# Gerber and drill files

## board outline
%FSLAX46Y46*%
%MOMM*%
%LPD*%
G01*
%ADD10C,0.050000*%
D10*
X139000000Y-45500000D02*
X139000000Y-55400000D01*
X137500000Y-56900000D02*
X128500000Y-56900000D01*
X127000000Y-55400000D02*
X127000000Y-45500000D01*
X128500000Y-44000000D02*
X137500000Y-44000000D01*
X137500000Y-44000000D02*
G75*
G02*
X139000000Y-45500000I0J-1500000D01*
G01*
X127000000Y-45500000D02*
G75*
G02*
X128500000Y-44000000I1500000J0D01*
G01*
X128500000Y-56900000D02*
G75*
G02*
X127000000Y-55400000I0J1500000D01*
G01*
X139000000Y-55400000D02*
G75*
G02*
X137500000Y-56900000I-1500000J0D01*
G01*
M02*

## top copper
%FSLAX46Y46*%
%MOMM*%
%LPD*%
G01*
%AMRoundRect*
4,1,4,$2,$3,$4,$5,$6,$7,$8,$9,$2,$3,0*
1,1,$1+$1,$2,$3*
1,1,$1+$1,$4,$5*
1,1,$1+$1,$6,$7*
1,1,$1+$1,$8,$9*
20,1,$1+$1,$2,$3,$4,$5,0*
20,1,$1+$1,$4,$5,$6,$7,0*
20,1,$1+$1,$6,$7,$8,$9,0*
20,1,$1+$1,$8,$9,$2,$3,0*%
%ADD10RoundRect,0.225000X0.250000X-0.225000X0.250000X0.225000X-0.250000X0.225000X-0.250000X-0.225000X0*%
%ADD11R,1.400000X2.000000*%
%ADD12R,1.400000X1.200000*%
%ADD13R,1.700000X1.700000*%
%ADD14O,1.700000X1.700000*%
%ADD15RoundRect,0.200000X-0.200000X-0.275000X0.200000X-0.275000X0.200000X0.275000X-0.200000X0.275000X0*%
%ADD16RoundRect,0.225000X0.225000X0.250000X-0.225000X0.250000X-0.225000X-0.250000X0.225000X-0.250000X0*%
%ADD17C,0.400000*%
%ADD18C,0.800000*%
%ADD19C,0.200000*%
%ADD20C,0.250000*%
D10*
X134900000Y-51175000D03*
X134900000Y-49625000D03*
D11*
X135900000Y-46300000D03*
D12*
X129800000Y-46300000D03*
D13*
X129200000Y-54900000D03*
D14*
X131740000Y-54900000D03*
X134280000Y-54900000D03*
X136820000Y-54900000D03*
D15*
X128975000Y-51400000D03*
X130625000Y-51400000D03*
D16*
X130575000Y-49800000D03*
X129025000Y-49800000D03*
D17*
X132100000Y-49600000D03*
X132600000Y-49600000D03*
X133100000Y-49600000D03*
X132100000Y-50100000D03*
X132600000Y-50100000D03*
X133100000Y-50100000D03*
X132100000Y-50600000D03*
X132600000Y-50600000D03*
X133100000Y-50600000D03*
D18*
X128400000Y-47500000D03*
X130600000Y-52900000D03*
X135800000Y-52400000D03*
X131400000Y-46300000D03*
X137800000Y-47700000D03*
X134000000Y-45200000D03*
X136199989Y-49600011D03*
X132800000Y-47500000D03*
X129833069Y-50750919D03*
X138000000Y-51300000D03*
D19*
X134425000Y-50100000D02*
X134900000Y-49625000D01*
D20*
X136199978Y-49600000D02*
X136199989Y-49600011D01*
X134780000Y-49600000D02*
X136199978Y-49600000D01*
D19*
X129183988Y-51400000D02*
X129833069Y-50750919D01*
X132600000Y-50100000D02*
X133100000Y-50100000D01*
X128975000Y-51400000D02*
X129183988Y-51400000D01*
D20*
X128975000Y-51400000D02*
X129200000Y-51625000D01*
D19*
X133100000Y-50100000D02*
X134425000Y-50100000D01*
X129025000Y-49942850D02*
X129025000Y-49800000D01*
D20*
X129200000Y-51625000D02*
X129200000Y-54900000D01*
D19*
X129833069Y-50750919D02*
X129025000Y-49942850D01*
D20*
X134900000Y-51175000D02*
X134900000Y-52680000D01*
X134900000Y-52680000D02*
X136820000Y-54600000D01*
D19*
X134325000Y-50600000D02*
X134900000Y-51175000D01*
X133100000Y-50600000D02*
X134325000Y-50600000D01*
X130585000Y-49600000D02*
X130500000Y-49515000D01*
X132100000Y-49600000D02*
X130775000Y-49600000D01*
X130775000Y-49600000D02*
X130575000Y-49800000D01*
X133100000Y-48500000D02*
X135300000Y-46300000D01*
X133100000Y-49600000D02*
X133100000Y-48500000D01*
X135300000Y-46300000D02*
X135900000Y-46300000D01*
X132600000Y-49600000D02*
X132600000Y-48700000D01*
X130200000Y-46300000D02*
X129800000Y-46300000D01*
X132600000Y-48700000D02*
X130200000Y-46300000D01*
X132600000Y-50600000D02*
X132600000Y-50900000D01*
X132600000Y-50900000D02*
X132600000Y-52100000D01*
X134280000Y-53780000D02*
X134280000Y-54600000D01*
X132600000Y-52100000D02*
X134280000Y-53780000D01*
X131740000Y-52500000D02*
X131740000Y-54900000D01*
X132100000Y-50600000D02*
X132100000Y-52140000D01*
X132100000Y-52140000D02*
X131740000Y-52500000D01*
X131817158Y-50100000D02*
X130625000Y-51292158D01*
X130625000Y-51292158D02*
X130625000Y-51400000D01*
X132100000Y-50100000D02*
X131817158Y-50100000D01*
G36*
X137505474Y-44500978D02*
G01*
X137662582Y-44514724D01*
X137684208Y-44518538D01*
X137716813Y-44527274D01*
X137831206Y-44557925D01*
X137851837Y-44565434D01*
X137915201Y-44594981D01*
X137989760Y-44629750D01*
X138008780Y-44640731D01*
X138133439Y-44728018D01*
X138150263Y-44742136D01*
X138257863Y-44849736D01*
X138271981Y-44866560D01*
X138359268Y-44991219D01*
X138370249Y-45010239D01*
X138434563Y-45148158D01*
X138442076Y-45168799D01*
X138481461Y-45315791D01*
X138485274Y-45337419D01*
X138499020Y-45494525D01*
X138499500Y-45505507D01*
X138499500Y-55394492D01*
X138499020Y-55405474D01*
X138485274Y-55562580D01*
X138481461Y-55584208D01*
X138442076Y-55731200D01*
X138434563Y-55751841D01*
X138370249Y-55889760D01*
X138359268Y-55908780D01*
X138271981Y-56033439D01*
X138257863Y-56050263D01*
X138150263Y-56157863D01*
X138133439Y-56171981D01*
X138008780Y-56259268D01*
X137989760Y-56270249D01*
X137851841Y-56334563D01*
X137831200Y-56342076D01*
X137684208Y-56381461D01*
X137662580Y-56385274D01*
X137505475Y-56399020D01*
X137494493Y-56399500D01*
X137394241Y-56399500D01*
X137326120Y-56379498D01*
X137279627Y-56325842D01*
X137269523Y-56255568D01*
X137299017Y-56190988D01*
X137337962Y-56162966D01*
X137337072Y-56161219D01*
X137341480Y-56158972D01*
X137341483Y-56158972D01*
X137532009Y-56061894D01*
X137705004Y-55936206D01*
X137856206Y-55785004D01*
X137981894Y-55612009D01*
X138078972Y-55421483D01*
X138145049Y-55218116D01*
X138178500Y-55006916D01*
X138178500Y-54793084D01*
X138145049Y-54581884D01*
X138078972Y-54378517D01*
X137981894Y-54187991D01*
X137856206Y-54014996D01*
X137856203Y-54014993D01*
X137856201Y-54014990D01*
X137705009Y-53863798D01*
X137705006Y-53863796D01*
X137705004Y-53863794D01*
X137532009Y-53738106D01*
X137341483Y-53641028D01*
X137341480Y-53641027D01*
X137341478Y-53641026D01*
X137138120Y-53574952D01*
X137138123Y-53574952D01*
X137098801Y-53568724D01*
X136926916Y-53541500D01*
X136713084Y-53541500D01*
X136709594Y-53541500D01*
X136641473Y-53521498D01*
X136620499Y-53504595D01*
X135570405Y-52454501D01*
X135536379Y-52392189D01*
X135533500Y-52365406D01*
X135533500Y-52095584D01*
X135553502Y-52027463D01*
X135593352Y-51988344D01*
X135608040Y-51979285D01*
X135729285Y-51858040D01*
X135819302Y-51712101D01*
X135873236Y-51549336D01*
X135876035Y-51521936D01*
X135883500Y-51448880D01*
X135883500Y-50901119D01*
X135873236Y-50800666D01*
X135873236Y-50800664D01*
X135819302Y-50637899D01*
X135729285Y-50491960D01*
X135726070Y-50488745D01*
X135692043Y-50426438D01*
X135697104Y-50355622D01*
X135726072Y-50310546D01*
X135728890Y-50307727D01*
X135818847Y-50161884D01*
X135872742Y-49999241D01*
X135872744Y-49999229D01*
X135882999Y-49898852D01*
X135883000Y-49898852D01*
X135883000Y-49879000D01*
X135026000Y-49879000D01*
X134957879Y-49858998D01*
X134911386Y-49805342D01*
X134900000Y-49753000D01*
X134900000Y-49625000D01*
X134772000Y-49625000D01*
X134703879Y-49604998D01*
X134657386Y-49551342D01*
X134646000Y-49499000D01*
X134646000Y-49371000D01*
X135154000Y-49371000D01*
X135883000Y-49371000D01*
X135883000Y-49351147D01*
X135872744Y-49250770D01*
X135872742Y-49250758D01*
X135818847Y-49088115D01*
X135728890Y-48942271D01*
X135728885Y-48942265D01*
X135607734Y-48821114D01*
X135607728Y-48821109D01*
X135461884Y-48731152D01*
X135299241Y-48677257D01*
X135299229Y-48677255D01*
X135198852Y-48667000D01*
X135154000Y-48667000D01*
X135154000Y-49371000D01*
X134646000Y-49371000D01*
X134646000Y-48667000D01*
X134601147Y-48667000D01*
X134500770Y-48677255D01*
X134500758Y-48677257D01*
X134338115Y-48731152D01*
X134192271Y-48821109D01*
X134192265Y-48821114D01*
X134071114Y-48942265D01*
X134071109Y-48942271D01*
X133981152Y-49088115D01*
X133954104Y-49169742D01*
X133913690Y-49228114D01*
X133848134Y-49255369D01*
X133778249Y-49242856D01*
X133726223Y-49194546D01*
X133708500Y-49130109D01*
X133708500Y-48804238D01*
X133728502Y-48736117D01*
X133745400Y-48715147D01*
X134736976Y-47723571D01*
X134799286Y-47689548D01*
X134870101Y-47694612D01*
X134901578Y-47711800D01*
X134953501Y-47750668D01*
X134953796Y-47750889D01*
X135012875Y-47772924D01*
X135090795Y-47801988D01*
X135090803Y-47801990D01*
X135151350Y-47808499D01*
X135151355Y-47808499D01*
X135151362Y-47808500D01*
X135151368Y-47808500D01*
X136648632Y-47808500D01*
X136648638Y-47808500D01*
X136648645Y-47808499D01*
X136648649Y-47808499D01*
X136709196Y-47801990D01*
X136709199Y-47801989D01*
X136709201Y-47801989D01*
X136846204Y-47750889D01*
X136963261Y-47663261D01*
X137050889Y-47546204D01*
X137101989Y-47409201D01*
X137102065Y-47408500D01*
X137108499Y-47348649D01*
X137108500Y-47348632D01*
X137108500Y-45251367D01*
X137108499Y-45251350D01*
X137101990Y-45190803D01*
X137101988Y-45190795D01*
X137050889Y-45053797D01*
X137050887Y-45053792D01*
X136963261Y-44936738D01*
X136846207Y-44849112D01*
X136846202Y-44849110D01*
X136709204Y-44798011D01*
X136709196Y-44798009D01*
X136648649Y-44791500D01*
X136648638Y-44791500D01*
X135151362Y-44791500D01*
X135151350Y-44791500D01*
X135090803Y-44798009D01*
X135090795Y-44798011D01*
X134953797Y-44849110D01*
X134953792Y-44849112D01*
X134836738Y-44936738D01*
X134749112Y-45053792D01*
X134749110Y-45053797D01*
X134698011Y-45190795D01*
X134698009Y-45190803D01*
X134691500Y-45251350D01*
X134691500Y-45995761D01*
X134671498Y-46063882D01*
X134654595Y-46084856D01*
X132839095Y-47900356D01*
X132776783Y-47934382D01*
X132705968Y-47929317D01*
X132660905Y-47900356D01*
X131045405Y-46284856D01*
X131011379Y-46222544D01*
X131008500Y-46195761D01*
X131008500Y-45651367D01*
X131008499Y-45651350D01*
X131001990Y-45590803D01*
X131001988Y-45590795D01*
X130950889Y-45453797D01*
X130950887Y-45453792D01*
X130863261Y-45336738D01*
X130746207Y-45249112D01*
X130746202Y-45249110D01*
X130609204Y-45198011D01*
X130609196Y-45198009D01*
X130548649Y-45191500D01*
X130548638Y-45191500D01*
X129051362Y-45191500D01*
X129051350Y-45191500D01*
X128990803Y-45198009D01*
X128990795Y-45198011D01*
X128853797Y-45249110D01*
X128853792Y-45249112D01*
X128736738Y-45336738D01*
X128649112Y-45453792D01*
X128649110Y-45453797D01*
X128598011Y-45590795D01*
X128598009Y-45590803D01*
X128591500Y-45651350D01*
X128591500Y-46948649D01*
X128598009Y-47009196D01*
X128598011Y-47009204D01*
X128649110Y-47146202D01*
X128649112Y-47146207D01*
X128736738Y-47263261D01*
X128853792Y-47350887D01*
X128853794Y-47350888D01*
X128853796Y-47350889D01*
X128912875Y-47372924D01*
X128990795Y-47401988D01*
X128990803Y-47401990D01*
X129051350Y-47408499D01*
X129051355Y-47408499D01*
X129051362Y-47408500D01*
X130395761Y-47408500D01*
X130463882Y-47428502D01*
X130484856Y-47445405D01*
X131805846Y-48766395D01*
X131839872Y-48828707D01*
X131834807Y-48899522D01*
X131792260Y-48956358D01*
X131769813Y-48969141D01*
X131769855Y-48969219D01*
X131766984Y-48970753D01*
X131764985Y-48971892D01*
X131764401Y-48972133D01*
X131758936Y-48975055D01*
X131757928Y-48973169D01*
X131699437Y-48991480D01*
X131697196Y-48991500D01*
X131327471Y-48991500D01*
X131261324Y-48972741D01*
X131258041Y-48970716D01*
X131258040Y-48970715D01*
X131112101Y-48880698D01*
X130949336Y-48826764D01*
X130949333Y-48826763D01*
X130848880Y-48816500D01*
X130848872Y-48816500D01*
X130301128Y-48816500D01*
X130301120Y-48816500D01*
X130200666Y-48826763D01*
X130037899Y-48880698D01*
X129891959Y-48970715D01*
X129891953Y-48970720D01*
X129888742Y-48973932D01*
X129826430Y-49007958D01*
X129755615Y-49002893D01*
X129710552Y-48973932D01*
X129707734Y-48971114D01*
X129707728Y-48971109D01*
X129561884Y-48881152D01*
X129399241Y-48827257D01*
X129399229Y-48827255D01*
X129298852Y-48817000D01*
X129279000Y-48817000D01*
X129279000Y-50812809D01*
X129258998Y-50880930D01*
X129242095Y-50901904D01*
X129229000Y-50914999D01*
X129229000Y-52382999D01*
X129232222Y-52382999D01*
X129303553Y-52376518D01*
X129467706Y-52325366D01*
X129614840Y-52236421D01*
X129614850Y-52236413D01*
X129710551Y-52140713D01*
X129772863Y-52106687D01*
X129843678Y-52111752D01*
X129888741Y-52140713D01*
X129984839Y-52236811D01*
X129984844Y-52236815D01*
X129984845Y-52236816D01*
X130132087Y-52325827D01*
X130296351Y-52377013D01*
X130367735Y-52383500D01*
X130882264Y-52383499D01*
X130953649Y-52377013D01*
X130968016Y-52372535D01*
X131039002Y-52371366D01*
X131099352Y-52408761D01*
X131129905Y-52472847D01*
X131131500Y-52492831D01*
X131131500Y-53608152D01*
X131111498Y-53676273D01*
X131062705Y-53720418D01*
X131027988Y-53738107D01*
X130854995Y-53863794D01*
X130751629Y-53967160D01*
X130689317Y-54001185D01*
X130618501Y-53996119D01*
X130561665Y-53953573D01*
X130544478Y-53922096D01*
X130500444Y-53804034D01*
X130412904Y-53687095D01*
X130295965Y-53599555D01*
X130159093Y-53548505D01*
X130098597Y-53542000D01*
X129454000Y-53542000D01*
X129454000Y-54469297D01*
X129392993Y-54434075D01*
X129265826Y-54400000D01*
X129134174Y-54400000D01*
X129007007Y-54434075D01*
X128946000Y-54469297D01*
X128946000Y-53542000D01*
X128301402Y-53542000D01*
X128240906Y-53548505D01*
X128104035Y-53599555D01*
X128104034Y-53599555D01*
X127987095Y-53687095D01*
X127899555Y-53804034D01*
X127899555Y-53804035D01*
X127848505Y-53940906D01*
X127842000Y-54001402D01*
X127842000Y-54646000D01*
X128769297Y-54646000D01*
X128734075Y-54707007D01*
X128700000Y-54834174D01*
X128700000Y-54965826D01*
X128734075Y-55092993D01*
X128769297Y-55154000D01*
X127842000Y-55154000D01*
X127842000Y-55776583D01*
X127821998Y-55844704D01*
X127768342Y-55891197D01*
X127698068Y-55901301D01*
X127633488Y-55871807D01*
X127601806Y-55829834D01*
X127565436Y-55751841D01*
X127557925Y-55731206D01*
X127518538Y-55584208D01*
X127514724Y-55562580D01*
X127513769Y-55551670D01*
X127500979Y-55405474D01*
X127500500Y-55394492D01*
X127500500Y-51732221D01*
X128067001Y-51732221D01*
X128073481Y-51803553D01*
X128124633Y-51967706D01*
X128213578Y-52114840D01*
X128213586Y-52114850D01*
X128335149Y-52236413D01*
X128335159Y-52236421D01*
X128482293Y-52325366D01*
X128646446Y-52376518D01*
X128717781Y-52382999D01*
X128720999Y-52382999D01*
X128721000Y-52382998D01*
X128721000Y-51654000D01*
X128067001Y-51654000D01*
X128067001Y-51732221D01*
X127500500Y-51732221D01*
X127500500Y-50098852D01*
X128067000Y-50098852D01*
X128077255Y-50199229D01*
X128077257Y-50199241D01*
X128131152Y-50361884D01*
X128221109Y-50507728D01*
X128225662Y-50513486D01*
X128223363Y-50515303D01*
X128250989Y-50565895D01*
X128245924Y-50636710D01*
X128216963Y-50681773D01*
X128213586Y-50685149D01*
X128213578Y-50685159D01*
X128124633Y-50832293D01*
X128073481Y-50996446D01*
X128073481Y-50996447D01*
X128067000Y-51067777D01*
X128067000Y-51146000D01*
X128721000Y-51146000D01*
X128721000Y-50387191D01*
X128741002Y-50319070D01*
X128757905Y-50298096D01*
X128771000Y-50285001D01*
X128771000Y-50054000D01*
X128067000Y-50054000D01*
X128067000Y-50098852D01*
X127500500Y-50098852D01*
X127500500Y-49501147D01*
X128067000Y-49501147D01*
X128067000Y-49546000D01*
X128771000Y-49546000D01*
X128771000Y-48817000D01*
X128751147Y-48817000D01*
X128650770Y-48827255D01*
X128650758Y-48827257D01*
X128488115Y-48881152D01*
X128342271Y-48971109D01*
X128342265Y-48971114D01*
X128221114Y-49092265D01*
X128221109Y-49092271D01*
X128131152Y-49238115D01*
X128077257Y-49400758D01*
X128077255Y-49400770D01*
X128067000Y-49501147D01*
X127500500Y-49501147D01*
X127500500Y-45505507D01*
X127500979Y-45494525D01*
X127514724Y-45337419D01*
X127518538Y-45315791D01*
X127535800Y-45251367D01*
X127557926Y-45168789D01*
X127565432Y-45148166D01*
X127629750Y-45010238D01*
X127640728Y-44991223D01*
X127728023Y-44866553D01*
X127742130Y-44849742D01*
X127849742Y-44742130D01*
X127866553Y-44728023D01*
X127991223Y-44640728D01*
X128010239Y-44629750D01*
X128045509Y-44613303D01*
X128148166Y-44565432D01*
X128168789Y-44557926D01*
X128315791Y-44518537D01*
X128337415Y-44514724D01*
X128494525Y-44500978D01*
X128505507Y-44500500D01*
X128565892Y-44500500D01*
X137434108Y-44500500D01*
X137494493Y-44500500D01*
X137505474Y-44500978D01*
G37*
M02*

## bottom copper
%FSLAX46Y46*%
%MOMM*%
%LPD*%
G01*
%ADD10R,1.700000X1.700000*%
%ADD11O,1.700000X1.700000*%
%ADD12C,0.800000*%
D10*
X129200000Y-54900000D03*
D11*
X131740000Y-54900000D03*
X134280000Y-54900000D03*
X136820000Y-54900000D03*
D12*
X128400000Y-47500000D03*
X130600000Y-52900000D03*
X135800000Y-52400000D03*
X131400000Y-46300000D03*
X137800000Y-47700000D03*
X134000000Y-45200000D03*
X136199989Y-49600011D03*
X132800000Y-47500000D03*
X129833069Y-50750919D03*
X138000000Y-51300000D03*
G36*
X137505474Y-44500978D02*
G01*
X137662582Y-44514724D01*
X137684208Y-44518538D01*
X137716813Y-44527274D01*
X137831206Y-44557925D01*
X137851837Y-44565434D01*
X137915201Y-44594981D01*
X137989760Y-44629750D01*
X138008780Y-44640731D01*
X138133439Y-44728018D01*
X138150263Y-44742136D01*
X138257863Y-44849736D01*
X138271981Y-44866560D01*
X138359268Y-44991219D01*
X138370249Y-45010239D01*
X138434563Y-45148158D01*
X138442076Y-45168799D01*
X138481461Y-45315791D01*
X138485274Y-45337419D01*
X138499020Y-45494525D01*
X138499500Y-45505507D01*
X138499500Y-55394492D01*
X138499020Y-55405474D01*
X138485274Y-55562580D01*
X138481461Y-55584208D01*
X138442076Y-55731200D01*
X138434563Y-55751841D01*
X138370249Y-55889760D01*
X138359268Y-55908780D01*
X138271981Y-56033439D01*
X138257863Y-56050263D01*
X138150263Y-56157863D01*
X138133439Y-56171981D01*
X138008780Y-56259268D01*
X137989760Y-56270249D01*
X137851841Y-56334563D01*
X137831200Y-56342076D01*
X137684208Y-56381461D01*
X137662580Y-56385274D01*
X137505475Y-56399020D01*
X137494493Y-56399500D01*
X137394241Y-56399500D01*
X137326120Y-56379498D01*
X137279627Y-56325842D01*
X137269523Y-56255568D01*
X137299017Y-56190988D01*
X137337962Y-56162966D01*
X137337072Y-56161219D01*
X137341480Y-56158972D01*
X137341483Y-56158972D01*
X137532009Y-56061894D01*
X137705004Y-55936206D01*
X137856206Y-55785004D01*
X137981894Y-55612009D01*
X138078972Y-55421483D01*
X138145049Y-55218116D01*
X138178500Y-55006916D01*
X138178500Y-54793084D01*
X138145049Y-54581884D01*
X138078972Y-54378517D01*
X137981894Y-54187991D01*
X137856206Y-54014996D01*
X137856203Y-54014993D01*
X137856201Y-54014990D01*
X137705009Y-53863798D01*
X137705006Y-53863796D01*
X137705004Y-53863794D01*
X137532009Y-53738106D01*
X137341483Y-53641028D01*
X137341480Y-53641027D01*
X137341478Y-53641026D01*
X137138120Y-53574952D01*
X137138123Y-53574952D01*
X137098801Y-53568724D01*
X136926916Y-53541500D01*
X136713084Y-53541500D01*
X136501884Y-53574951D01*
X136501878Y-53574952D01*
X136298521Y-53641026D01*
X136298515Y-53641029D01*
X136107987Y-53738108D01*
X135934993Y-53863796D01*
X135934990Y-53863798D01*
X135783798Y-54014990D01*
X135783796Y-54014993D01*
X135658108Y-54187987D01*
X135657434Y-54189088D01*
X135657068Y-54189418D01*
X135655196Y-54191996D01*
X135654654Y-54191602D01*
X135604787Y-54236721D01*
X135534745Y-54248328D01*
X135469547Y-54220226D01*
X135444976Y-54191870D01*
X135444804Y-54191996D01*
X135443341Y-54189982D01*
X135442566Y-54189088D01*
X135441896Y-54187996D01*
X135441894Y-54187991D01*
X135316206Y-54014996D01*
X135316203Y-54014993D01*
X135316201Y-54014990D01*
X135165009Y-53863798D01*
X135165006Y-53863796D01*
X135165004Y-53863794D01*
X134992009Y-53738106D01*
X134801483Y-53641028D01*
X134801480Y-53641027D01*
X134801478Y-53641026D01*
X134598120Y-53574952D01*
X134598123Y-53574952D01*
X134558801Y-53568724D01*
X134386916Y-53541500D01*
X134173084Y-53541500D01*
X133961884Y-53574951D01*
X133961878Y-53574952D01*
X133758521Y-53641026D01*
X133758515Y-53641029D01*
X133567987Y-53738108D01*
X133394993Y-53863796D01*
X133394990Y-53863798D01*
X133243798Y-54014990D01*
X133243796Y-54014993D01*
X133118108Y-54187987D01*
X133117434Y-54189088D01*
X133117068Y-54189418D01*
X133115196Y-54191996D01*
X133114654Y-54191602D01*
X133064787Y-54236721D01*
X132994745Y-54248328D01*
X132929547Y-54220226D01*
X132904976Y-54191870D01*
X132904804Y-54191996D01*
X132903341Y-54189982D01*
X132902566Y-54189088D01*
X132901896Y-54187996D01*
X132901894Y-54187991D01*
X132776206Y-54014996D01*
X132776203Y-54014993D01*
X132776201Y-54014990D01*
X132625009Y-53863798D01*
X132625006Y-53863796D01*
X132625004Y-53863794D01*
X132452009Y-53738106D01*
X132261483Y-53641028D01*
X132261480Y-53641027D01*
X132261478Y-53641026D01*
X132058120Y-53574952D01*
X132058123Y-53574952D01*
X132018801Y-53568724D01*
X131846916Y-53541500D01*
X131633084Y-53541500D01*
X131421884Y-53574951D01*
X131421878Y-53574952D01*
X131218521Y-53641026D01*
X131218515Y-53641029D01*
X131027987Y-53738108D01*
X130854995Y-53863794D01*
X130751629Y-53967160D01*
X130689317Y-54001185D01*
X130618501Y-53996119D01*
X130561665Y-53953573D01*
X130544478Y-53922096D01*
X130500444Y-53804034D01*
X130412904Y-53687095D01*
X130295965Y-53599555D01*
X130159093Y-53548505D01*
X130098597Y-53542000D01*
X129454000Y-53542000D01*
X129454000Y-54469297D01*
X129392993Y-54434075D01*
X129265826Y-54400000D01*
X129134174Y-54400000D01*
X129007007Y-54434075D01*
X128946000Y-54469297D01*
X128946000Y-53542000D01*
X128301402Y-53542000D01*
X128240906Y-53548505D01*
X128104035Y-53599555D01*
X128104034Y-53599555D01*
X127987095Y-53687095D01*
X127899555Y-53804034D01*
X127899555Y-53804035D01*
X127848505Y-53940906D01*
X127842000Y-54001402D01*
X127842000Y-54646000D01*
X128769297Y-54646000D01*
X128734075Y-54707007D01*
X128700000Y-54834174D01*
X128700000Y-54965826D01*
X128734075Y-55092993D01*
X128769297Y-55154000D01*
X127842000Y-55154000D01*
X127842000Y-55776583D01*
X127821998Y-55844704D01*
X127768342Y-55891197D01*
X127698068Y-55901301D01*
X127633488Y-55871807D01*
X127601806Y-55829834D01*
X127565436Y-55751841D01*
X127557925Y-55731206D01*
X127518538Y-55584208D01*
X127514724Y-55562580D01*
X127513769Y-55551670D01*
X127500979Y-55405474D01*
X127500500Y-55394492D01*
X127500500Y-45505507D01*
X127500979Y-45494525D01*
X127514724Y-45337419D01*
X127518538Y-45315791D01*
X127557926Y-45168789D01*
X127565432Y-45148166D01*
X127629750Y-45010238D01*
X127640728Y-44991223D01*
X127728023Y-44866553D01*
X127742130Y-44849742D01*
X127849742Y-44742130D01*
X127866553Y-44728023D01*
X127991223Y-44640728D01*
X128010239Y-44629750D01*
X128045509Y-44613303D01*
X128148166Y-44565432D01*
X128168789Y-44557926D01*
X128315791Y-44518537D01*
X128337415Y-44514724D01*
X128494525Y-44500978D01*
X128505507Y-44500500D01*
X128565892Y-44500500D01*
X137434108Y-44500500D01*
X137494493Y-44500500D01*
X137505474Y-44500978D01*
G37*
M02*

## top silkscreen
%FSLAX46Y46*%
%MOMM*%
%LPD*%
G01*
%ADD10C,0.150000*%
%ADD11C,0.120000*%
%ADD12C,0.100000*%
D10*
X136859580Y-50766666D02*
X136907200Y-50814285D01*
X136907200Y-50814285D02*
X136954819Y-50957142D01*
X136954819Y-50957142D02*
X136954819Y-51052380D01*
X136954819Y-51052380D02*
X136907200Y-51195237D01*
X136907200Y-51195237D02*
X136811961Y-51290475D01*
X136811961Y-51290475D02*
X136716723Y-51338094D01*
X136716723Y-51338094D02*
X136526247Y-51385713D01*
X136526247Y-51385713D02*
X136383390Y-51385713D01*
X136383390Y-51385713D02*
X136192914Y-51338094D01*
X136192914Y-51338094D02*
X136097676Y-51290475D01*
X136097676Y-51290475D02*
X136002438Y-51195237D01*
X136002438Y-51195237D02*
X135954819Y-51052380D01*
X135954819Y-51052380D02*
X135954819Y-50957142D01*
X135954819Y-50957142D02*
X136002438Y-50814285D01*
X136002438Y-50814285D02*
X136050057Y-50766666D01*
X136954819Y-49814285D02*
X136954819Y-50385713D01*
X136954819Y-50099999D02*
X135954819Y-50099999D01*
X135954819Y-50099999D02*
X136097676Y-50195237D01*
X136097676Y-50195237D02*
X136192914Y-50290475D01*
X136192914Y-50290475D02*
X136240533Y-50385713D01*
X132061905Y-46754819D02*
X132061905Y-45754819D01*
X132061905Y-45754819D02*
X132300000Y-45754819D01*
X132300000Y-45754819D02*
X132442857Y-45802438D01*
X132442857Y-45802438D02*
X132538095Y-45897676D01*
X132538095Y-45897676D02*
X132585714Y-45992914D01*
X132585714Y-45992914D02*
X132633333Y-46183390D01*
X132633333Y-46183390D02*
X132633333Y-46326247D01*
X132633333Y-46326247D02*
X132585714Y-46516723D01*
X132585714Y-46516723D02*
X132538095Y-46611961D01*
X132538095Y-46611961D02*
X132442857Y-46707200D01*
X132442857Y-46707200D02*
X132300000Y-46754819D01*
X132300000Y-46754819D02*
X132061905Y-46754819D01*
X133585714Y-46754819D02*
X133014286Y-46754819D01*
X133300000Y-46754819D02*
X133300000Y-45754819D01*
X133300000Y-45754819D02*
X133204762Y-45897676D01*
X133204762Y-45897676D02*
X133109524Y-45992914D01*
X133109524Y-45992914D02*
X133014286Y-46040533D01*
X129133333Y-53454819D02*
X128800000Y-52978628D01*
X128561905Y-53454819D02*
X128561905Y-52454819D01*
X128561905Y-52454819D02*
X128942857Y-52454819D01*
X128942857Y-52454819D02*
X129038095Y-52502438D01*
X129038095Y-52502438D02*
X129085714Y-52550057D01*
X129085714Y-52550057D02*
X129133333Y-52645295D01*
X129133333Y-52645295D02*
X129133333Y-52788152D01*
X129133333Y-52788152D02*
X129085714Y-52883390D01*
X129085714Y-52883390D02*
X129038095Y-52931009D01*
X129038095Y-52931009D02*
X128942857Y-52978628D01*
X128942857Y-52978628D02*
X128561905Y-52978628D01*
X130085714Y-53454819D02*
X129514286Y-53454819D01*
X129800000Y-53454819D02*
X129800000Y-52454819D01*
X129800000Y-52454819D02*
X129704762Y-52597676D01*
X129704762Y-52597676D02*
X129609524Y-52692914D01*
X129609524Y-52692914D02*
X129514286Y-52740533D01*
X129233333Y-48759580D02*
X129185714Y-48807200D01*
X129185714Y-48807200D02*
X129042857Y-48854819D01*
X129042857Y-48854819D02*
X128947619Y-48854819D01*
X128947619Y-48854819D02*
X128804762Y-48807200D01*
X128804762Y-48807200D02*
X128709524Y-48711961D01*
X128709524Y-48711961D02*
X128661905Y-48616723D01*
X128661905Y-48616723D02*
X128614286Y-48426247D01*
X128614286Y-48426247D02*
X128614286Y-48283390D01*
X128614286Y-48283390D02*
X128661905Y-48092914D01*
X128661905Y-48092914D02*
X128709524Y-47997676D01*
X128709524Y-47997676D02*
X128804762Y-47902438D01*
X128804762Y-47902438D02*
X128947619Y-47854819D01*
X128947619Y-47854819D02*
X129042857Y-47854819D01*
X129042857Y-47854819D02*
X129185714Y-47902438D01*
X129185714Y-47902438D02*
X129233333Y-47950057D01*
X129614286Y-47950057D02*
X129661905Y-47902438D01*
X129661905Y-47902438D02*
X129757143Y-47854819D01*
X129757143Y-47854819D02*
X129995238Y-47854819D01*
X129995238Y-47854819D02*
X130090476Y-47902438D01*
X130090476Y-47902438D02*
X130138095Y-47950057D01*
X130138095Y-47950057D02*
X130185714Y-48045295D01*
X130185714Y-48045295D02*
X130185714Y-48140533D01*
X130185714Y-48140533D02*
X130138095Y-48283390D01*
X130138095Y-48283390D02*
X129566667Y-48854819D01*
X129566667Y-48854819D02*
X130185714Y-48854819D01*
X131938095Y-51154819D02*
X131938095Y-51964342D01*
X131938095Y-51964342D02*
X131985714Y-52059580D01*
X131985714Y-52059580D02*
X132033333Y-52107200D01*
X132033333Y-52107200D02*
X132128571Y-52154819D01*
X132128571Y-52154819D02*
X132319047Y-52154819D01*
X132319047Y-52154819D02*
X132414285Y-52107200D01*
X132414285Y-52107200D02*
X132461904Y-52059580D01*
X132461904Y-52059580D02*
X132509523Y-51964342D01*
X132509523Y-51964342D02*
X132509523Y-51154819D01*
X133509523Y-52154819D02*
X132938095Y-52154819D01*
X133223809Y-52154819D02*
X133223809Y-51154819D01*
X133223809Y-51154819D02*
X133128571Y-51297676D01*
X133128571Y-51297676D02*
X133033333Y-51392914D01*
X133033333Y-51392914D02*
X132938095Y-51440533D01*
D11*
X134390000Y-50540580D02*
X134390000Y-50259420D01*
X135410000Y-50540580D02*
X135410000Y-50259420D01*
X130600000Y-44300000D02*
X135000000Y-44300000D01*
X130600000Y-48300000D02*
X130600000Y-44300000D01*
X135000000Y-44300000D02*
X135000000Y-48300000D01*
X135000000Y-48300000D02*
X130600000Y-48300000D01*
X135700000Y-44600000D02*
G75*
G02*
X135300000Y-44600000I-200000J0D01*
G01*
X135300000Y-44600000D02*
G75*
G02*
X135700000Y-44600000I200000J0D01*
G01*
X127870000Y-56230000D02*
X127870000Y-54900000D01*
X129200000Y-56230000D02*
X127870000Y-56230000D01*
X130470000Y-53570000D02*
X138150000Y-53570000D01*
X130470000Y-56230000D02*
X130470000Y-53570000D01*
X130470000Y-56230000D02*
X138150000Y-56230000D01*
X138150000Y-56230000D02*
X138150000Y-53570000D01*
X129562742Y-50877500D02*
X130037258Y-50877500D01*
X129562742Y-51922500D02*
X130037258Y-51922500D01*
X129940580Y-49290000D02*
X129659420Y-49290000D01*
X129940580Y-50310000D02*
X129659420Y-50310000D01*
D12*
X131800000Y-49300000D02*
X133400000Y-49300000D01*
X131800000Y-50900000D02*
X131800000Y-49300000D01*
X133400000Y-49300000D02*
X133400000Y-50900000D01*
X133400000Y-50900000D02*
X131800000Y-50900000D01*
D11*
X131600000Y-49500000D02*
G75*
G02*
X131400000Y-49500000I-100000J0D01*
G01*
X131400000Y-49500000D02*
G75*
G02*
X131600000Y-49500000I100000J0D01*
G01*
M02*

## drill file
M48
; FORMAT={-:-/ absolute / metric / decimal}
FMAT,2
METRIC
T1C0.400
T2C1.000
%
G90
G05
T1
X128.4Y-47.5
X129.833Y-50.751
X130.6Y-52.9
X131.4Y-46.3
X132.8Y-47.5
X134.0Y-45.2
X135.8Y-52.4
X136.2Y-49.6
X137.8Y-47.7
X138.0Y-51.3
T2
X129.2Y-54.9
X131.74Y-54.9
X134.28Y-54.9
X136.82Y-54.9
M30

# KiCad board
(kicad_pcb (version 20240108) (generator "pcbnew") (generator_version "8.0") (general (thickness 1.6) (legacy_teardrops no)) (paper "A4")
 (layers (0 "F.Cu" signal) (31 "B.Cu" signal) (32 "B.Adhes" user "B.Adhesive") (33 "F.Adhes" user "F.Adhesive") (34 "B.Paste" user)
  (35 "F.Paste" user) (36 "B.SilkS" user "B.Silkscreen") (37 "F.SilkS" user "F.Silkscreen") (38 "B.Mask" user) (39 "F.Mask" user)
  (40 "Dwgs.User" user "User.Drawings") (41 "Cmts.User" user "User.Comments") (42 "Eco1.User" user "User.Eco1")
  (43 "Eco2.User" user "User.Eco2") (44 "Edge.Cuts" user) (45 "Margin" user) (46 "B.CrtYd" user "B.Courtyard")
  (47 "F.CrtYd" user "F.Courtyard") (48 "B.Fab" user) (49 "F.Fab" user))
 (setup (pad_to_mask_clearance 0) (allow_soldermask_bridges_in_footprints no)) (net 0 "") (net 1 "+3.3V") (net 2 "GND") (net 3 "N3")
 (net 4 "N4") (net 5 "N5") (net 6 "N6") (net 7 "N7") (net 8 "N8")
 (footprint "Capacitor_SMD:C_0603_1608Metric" (layer "F.Cu") (at 134.9 50.4 90)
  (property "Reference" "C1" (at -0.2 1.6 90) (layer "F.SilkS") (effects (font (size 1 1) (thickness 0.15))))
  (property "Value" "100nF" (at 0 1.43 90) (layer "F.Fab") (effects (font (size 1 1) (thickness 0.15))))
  (fp_line (start -0.14058 -0.51) (end 0.14058 -0.51) (stroke (width 0.12) (type solid)) (layer "F.SilkS"))
  (fp_line (start -0.14058 0.51) (end 0.14058 0.51) (stroke (width 0.12) (type solid)) (layer "F.SilkS"))
  (pad "1" smd roundrect (at -0.775 0 90) (size 0.9 0.95) (layers "F.Cu" "F.Paste" "F.Mask") (roundrect_rratio 0.25) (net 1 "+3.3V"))
  (pad "2" smd roundrect (at 0.775 0 90) (size 0.9 0.95) (layers "F.Cu" "F.Paste" "F.Mask") (roundrect_rratio 0.25) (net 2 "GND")))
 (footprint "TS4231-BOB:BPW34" (layer "F.Cu") (at 132.8 46.3)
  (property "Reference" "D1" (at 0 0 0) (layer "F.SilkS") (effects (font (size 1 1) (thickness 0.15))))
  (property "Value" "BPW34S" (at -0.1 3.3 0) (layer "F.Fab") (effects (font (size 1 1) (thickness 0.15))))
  (fp_line (start -2.2 -2) (end 2.2 -2) (stroke (width 0.12) (type solid)) (layer "F.SilkS"))
  (fp_line (start -2.2 2) (end -2.2 -2) (stroke (width 0.12) (type solid)) (layer "F.SilkS"))
  (fp_line (start 2.2 -2) (end 2.2 2) (stroke (width 0.12) (type solid)) (layer "F.SilkS"))
  (fp_line (start 2.2 2) (end -2.2 2) (stroke (width 0.12) (type solid)) (layer "F.SilkS"))
  (fp_circle (center 2.7 -1.7) (end 2.9 -1.7) (stroke (width 0.12) (type solid)) (fill none) (layer "F.SilkS"))
  (pad "1" smd rect (at 3.1 0) (size 1.4 2) (layers "F.Cu" "F.Paste" "F.Mask") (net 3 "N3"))
  (pad "2" smd rect (at -3 0) (size 1.4 1.2) (layers "F.Cu" "F.Paste" "F.Mask") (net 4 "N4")))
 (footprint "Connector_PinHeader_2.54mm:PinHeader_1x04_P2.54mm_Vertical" (layer "F.Cu") (at 129.2 54.9 90)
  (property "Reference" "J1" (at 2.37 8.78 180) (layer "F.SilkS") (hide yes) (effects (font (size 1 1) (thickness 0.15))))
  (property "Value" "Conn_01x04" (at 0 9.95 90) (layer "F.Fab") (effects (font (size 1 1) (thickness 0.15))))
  (fp_line (start -1.33 -1.33) (end 0 -1.33) (stroke (width 0.12) (type solid)) (layer "F.SilkS"))
  (fp_line (start -1.33 0) (end -1.33 -1.33) (stroke (width 0.12) (type solid)) (layer "F.SilkS"))
  (fp_line (start 1.33 1.27) (end 1.33 8.95) (stroke (width 0.12) (type solid)) (layer "F.SilkS"))
  (fp_line (start -1.33 1.27) (end 1.33 1.27) (stroke (width 0.12) (type solid)) (layer "F.SilkS"))
  (fp_line (start -1.33 1.27) (end -1.33 8.95) (stroke (width 0.12) (type solid)) (layer "F.SilkS"))
  (fp_line (start -1.33 8.95) (end 1.33 8.95) (stroke (width 0.12) (type solid)) (layer "F.SilkS"))
  (pad "1" thru_hole rect (at 0 0 90) (size 1.7 1.7) (drill 1) (layers "*.Cu" "*.Mask") (remove_unused_layers no) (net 2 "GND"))
  (pad "2" thru_hole oval (at 0 2.54 90) (size 1.7 1.7) (drill 1) (layers "*.Cu" "*.Mask") (remove_unused_layers no) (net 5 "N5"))
  (pad "3" thru_hole oval (at 0 5.08 90) (size 1.7 1.7) (drill 1) (layers "*.Cu" "*.Mask") (remove_unused_layers no) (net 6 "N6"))
  (pad "4" thru_hole oval (at 0 7.62 90) (size 1.7 1.7) (drill 1) (layers "*.Cu" "*.Mask") (remove_unused_layers no) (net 1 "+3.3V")))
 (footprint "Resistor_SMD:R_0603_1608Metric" (layer "F.Cu") (at 129.8 51.4)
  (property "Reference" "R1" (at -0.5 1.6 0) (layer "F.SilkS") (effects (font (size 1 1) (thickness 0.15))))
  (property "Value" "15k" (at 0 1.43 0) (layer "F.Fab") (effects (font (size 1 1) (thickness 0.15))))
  (fp_line (start -0.237258 -0.5225) (end 0.237258 -0.5225) (stroke (width 0.12) (type solid)) (layer "F.SilkS"))
  (fp_line (start -0.237258 0.5225) (end 0.237258 0.5225) (stroke (width 0.12) (type solid)) (layer "F.SilkS"))
  (pad "1" smd roundrect (at -0.825 0) (size 0.8 0.95) (layers "F.Cu" "F.Paste" "F.Mask") (roundrect_rratio 0.25) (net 2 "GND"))
  (pad "2" smd roundrect (at 0.825 0) (size 0.8 0.95) (layers "F.Cu" "F.Paste" "F.Mask") (roundrect_rratio 0.25) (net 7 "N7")))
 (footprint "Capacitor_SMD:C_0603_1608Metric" (layer "F.Cu") (at 129.8 49.8 180)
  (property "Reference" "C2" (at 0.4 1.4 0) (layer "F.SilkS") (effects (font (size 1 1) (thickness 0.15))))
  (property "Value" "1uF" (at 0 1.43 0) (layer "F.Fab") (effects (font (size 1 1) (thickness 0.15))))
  (fp_line (start -0.14058 0.51) (end 0.14058 0.51) (stroke (width 0.12) (type solid)) (layer "F.SilkS"))
  (fp_line (start -0.14058 -0.51) (end 0.14058 -0.51) (stroke (width 0.12) (type solid)) (layer "F.SilkS"))
  (pad "1" smd roundrect (at -0.775 0 180) (size 0.9 0.95) (layers "F.Cu" "F.Paste" "F.Mask") (roundrect_rratio 0.25) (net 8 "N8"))
  (pad "2" smd roundrect (at 0.775 0 180) (size 0.9 0.95) (layers "F.Cu" "F.Paste" "F.Mask") (roundrect_rratio 0.25) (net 2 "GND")))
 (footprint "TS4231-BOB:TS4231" (layer "F.Cu") (at 132.6 50.1)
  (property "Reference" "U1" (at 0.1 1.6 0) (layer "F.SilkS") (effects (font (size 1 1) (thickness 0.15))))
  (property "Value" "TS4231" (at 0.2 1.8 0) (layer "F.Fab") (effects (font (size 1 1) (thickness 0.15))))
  (fp_line (start -0.8 -0.8) (end 0.8 -0.8) (stroke (width 0.1) (type solid)) (layer "F.SilkS"))
  (fp_line (start -0.8 0.8) (end -0.8 -0.8) (stroke (width 0.1) (type solid)) (layer "F.SilkS"))
  (fp_line (start 0.8 -0.8) (end 0.8 0.8) (stroke (width 0.1) (type solid)) (layer "F.SilkS"))
  (fp_line (start 0.8 0.8) (end -0.8 0.8) (stroke (width 0.1) (type solid)) (layer "F.SilkS"))
  (fp_circle (center -1.1 -0.6) (end -1 -0.6) (stroke (width 0.12) (type solid)) (fill none) (layer "F.SilkS"))
  (pad "A1" smd circle (at -0.5 -0.5) (size 0.4 0.4) (layers "F.Cu" "F.Paste" "F.Mask") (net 8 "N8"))
  (pad "A2" smd circle (at 0 -0.5) (size 0.4 0.4) (layers "F.Cu" "F.Paste" "F.Mask") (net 4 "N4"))
  (pad "A3" smd circle (at 0.5 -0.5) (size 0.4 0.4) (layers "F.Cu" "F.Paste" "F.Mask") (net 3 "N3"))
  (pad "B1" smd circle (at -0.5 0) (size 0.4 0.4) (layers "F.Cu" "F.Paste" "F.Mask") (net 7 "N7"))
  (pad "B2" smd circle (at 0 0) (size 0.4 0.4) (layers "F.Cu" "F.Paste" "F.Mask") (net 2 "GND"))
  (pad "B3" smd circle (at 0.5 0) (size 0.4 0.4) (layers "F.Cu" "F.Paste" "F.Mask") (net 2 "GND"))
  (pad "C1" smd circle (at -0.5 0.5) (size 0.4 0.4) (layers "F.Cu" "F.Paste" "F.Mask") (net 5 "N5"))
  (pad "C2" smd circle (at 0 0.5) (size 0.4 0.4) (layers "F.Cu" "F.Paste" "F.Mask") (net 6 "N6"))
  (pad "C3" smd circle (at 0.5 0.5) (size 0.4 0.4) (layers "F.Cu" "F.Paste" "F.Mask") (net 1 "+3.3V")))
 (gr_line (start 139 45.5) (end 139 55.4) (stroke (width 0.05) (type solid)) (layer "Edge.Cuts"))
 (gr_line (start 137.5 56.9) (end 128.5 56.9) (stroke (width 0.05) (type solid)) (layer "Edge.Cuts"))
 (gr_line (start 127 55.4) (end 127 45.5) (stroke (width 0.05) (type solid)) (layer "Edge.Cuts"))
 (gr_line (start 128.5 44) (end 137.5 44) (stroke (width 0.05) (type solid)) (layer "Edge.Cuts"))
 (gr_arc (start 137.5 44) (mid 138.56066 44.43934) (end 139 45.5) (stroke (width 0.05) (type solid)) (layer "Edge.Cuts"))
 (gr_arc (start 127 45.5) (mid 127.43934 44.43934) (end 128.5 44) (stroke (width 0.05) (type solid)) (layer "Edge.Cuts"))
 (gr_arc (start 128.5 56.9) (mid 127.43934 56.46066) (end 127 55.4) (stroke (width 0.05) (type solid)) (layer "Edge.Cuts"))
 (gr_arc (start 139 55.4) (mid 138.56066 56.46066) (end 137.5 56.9) (stroke (width 0.05) (type solid)) (layer "Edge.Cuts"))
 (segment (start 134.425 50.1) (end 134.9 49.625) (width 0.2) (layer "F.Cu") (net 2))
 (segment (start 136.199978 49.6) (end 136.199989 49.600011) (width 0.25) (layer "F.Cu") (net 2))
 (segment (start 134.78 49.6) (end 136.199978 49.6) (width 0.25) (layer "F.Cu") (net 2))
 (segment (start 129.183988 51.4) (end 129.833069 50.750919) (width 0.2) (layer "F.Cu") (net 2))
 (segment (start 132.6 50.1) (end 133.1 50.1) (width 0.2) (layer "F.Cu") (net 2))
 (segment (start 128.975 51.4) (end 129.183988 51.4) (width 0.2) (layer "F.Cu") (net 2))
 (segment (start 128.975 51.4) (end 129.2 51.625) (width 0.25) (layer "F.Cu") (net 2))
 (segment (start 133.1 50.1) (end 134.425 50.1) (width 0.2) (layer "F.Cu") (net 2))
 (segment (start 129.025 49.94285) (end 129.025 49.8) (width 0.2) (layer "F.Cu") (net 2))
 (segment (start 129.2 51.625) (end 129.2 54.9) (width 0.25) (layer "F.Cu") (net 2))
 (segment (start 129.833069 50.750919) (end 129.025 49.94285) (width 0.2) (layer "F.Cu") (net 2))
 (via (at 128.4 47.5) (size 0.8) (drill 0.4) (layers "F.Cu" "B.Cu") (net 2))
 (via (at 130.6 52.9) (size 0.8) (drill 0.4) (layers "F.Cu" "B.Cu") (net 2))
 (via (at 135.8 52.4) (size 0.8) (drill 0.4) (layers "F.Cu" "B.Cu") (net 2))
 (via (at 131.4 46.3) (size 0.8) (drill 0.4) (layers "F.Cu" "B.Cu") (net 2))
 (via (at 137.8 47.7) (size 0.8) (drill 0.4) (layers "F.Cu" "B.Cu") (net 2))
 (via (at 134 45.2) (size 0.8) (drill 0.4) (layers "F.Cu" "B.Cu") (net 2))
 (via (at 136.199989 49.600011) (size 0.8) (drill 0.4) (layers "F.Cu" "B.Cu") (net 2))
 (via (at 132.8 47.5) (size 0.8) (drill 0.4) (layers "F.Cu" "B.Cu") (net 2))
 (via (at 129.833069 50.750919) (size 0.8) (drill 0.4) (layers "F.Cu" "B.Cu") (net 2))
 (via (at 138 51.3) (size 0.8) (drill 0.4) (layers "F.Cu" "B.Cu") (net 2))
 (segment (start 134.9 51.175) (end 134.9 52.68) (width 0.25) (layer "F.Cu") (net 1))
 (segment (start 134.9 52.68) (end 136.82 54.6) (width 0.25) (layer "F.Cu") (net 1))
 (segment (start 134.325 50.6) (end 134.9 51.175) (width 0.2) (layer "F.Cu") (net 1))
 (segment (start 133.1 50.6) (end 134.325 50.6) (width 0.2) (layer "F.Cu") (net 1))
 (segment (start 130.585 49.6) (end 130.5 49.515) (width 0.2) (layer "F.Cu") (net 8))
 (segment (start 132.1 49.6) (end 130.775 49.6) (width 0.2) (layer "F.Cu") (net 8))
 (segment (start 130.775 49.6) (end 130.575 49.8) (width 0.2) (layer "F.Cu") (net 8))
 (segment (start 133.1 48.5) (end 135.3 46.3) (width 0.2) (layer "F.Cu") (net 3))
 (segment (start 133.1 49.6) (end 133.1 48.5) (width 0.2) (layer "F.Cu") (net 3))
 (segment (start 135.3 46.3) (end 135.9 46.3) (width 0.2) (layer "F.Cu") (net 3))
 (segment (start 132.6 49.6) (end 132.6 48.7) (width 0.2) (layer "F.Cu") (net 4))
 (segment (start 130.2 46.3) (end 129.8 46.3) (width 0.2) (layer "F.Cu") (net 4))
 (segment (start 132.6 48.7) (end 130.2 46.3) (width 0.2) (layer "F.Cu") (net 4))
 (segment (start 132.6 50.6) (end 132.6 50.9) (width 0.2) (layer "F.Cu") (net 6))
 (segment (start 132.6 50.9) (end 132.6 52.1) (width 0.2) (layer "F.Cu") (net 6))
 (segment (start 134.28 53.78) (end 134.28 54.6) (width 0.2) (layer "F.Cu") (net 6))
 (segment (start 132.6 52.1) (end 134.28 53.78) (width 0.2) (layer "F.Cu") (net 6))
 (segment (start 131.74 52.5) (end 131.74 54.9) (width 0.2) (layer "F.Cu") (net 5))
 (segment (start 132.1 50.6) (end 132.1 52.14) (width 0.2) (layer "F.Cu") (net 5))
 (segment (start 132.1 52.14) (end 131.74 52.5) (width 0.2) (layer "F.Cu") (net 5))
 (segment (start 131.817158 50.1) (end 130.625 51.292158) (width 0.2) (layer "F.Cu") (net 7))
 (segment (start 130.625 51.292158) (end 130.625 51.4) (width 0.2) (layer "F.Cu") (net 7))
 (segment (start 132.1 50.1) (end 131.817158 50.1) (width 0.2) (layer "F.Cu") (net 7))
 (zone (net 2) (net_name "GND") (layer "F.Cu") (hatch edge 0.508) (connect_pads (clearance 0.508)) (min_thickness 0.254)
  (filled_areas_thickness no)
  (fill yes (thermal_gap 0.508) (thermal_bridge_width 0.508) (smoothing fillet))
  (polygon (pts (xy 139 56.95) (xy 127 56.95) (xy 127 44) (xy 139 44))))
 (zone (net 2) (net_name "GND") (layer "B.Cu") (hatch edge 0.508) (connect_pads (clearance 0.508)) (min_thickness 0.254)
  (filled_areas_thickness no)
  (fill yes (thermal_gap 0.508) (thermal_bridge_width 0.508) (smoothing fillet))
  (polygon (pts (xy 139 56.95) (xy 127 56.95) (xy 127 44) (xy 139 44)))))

